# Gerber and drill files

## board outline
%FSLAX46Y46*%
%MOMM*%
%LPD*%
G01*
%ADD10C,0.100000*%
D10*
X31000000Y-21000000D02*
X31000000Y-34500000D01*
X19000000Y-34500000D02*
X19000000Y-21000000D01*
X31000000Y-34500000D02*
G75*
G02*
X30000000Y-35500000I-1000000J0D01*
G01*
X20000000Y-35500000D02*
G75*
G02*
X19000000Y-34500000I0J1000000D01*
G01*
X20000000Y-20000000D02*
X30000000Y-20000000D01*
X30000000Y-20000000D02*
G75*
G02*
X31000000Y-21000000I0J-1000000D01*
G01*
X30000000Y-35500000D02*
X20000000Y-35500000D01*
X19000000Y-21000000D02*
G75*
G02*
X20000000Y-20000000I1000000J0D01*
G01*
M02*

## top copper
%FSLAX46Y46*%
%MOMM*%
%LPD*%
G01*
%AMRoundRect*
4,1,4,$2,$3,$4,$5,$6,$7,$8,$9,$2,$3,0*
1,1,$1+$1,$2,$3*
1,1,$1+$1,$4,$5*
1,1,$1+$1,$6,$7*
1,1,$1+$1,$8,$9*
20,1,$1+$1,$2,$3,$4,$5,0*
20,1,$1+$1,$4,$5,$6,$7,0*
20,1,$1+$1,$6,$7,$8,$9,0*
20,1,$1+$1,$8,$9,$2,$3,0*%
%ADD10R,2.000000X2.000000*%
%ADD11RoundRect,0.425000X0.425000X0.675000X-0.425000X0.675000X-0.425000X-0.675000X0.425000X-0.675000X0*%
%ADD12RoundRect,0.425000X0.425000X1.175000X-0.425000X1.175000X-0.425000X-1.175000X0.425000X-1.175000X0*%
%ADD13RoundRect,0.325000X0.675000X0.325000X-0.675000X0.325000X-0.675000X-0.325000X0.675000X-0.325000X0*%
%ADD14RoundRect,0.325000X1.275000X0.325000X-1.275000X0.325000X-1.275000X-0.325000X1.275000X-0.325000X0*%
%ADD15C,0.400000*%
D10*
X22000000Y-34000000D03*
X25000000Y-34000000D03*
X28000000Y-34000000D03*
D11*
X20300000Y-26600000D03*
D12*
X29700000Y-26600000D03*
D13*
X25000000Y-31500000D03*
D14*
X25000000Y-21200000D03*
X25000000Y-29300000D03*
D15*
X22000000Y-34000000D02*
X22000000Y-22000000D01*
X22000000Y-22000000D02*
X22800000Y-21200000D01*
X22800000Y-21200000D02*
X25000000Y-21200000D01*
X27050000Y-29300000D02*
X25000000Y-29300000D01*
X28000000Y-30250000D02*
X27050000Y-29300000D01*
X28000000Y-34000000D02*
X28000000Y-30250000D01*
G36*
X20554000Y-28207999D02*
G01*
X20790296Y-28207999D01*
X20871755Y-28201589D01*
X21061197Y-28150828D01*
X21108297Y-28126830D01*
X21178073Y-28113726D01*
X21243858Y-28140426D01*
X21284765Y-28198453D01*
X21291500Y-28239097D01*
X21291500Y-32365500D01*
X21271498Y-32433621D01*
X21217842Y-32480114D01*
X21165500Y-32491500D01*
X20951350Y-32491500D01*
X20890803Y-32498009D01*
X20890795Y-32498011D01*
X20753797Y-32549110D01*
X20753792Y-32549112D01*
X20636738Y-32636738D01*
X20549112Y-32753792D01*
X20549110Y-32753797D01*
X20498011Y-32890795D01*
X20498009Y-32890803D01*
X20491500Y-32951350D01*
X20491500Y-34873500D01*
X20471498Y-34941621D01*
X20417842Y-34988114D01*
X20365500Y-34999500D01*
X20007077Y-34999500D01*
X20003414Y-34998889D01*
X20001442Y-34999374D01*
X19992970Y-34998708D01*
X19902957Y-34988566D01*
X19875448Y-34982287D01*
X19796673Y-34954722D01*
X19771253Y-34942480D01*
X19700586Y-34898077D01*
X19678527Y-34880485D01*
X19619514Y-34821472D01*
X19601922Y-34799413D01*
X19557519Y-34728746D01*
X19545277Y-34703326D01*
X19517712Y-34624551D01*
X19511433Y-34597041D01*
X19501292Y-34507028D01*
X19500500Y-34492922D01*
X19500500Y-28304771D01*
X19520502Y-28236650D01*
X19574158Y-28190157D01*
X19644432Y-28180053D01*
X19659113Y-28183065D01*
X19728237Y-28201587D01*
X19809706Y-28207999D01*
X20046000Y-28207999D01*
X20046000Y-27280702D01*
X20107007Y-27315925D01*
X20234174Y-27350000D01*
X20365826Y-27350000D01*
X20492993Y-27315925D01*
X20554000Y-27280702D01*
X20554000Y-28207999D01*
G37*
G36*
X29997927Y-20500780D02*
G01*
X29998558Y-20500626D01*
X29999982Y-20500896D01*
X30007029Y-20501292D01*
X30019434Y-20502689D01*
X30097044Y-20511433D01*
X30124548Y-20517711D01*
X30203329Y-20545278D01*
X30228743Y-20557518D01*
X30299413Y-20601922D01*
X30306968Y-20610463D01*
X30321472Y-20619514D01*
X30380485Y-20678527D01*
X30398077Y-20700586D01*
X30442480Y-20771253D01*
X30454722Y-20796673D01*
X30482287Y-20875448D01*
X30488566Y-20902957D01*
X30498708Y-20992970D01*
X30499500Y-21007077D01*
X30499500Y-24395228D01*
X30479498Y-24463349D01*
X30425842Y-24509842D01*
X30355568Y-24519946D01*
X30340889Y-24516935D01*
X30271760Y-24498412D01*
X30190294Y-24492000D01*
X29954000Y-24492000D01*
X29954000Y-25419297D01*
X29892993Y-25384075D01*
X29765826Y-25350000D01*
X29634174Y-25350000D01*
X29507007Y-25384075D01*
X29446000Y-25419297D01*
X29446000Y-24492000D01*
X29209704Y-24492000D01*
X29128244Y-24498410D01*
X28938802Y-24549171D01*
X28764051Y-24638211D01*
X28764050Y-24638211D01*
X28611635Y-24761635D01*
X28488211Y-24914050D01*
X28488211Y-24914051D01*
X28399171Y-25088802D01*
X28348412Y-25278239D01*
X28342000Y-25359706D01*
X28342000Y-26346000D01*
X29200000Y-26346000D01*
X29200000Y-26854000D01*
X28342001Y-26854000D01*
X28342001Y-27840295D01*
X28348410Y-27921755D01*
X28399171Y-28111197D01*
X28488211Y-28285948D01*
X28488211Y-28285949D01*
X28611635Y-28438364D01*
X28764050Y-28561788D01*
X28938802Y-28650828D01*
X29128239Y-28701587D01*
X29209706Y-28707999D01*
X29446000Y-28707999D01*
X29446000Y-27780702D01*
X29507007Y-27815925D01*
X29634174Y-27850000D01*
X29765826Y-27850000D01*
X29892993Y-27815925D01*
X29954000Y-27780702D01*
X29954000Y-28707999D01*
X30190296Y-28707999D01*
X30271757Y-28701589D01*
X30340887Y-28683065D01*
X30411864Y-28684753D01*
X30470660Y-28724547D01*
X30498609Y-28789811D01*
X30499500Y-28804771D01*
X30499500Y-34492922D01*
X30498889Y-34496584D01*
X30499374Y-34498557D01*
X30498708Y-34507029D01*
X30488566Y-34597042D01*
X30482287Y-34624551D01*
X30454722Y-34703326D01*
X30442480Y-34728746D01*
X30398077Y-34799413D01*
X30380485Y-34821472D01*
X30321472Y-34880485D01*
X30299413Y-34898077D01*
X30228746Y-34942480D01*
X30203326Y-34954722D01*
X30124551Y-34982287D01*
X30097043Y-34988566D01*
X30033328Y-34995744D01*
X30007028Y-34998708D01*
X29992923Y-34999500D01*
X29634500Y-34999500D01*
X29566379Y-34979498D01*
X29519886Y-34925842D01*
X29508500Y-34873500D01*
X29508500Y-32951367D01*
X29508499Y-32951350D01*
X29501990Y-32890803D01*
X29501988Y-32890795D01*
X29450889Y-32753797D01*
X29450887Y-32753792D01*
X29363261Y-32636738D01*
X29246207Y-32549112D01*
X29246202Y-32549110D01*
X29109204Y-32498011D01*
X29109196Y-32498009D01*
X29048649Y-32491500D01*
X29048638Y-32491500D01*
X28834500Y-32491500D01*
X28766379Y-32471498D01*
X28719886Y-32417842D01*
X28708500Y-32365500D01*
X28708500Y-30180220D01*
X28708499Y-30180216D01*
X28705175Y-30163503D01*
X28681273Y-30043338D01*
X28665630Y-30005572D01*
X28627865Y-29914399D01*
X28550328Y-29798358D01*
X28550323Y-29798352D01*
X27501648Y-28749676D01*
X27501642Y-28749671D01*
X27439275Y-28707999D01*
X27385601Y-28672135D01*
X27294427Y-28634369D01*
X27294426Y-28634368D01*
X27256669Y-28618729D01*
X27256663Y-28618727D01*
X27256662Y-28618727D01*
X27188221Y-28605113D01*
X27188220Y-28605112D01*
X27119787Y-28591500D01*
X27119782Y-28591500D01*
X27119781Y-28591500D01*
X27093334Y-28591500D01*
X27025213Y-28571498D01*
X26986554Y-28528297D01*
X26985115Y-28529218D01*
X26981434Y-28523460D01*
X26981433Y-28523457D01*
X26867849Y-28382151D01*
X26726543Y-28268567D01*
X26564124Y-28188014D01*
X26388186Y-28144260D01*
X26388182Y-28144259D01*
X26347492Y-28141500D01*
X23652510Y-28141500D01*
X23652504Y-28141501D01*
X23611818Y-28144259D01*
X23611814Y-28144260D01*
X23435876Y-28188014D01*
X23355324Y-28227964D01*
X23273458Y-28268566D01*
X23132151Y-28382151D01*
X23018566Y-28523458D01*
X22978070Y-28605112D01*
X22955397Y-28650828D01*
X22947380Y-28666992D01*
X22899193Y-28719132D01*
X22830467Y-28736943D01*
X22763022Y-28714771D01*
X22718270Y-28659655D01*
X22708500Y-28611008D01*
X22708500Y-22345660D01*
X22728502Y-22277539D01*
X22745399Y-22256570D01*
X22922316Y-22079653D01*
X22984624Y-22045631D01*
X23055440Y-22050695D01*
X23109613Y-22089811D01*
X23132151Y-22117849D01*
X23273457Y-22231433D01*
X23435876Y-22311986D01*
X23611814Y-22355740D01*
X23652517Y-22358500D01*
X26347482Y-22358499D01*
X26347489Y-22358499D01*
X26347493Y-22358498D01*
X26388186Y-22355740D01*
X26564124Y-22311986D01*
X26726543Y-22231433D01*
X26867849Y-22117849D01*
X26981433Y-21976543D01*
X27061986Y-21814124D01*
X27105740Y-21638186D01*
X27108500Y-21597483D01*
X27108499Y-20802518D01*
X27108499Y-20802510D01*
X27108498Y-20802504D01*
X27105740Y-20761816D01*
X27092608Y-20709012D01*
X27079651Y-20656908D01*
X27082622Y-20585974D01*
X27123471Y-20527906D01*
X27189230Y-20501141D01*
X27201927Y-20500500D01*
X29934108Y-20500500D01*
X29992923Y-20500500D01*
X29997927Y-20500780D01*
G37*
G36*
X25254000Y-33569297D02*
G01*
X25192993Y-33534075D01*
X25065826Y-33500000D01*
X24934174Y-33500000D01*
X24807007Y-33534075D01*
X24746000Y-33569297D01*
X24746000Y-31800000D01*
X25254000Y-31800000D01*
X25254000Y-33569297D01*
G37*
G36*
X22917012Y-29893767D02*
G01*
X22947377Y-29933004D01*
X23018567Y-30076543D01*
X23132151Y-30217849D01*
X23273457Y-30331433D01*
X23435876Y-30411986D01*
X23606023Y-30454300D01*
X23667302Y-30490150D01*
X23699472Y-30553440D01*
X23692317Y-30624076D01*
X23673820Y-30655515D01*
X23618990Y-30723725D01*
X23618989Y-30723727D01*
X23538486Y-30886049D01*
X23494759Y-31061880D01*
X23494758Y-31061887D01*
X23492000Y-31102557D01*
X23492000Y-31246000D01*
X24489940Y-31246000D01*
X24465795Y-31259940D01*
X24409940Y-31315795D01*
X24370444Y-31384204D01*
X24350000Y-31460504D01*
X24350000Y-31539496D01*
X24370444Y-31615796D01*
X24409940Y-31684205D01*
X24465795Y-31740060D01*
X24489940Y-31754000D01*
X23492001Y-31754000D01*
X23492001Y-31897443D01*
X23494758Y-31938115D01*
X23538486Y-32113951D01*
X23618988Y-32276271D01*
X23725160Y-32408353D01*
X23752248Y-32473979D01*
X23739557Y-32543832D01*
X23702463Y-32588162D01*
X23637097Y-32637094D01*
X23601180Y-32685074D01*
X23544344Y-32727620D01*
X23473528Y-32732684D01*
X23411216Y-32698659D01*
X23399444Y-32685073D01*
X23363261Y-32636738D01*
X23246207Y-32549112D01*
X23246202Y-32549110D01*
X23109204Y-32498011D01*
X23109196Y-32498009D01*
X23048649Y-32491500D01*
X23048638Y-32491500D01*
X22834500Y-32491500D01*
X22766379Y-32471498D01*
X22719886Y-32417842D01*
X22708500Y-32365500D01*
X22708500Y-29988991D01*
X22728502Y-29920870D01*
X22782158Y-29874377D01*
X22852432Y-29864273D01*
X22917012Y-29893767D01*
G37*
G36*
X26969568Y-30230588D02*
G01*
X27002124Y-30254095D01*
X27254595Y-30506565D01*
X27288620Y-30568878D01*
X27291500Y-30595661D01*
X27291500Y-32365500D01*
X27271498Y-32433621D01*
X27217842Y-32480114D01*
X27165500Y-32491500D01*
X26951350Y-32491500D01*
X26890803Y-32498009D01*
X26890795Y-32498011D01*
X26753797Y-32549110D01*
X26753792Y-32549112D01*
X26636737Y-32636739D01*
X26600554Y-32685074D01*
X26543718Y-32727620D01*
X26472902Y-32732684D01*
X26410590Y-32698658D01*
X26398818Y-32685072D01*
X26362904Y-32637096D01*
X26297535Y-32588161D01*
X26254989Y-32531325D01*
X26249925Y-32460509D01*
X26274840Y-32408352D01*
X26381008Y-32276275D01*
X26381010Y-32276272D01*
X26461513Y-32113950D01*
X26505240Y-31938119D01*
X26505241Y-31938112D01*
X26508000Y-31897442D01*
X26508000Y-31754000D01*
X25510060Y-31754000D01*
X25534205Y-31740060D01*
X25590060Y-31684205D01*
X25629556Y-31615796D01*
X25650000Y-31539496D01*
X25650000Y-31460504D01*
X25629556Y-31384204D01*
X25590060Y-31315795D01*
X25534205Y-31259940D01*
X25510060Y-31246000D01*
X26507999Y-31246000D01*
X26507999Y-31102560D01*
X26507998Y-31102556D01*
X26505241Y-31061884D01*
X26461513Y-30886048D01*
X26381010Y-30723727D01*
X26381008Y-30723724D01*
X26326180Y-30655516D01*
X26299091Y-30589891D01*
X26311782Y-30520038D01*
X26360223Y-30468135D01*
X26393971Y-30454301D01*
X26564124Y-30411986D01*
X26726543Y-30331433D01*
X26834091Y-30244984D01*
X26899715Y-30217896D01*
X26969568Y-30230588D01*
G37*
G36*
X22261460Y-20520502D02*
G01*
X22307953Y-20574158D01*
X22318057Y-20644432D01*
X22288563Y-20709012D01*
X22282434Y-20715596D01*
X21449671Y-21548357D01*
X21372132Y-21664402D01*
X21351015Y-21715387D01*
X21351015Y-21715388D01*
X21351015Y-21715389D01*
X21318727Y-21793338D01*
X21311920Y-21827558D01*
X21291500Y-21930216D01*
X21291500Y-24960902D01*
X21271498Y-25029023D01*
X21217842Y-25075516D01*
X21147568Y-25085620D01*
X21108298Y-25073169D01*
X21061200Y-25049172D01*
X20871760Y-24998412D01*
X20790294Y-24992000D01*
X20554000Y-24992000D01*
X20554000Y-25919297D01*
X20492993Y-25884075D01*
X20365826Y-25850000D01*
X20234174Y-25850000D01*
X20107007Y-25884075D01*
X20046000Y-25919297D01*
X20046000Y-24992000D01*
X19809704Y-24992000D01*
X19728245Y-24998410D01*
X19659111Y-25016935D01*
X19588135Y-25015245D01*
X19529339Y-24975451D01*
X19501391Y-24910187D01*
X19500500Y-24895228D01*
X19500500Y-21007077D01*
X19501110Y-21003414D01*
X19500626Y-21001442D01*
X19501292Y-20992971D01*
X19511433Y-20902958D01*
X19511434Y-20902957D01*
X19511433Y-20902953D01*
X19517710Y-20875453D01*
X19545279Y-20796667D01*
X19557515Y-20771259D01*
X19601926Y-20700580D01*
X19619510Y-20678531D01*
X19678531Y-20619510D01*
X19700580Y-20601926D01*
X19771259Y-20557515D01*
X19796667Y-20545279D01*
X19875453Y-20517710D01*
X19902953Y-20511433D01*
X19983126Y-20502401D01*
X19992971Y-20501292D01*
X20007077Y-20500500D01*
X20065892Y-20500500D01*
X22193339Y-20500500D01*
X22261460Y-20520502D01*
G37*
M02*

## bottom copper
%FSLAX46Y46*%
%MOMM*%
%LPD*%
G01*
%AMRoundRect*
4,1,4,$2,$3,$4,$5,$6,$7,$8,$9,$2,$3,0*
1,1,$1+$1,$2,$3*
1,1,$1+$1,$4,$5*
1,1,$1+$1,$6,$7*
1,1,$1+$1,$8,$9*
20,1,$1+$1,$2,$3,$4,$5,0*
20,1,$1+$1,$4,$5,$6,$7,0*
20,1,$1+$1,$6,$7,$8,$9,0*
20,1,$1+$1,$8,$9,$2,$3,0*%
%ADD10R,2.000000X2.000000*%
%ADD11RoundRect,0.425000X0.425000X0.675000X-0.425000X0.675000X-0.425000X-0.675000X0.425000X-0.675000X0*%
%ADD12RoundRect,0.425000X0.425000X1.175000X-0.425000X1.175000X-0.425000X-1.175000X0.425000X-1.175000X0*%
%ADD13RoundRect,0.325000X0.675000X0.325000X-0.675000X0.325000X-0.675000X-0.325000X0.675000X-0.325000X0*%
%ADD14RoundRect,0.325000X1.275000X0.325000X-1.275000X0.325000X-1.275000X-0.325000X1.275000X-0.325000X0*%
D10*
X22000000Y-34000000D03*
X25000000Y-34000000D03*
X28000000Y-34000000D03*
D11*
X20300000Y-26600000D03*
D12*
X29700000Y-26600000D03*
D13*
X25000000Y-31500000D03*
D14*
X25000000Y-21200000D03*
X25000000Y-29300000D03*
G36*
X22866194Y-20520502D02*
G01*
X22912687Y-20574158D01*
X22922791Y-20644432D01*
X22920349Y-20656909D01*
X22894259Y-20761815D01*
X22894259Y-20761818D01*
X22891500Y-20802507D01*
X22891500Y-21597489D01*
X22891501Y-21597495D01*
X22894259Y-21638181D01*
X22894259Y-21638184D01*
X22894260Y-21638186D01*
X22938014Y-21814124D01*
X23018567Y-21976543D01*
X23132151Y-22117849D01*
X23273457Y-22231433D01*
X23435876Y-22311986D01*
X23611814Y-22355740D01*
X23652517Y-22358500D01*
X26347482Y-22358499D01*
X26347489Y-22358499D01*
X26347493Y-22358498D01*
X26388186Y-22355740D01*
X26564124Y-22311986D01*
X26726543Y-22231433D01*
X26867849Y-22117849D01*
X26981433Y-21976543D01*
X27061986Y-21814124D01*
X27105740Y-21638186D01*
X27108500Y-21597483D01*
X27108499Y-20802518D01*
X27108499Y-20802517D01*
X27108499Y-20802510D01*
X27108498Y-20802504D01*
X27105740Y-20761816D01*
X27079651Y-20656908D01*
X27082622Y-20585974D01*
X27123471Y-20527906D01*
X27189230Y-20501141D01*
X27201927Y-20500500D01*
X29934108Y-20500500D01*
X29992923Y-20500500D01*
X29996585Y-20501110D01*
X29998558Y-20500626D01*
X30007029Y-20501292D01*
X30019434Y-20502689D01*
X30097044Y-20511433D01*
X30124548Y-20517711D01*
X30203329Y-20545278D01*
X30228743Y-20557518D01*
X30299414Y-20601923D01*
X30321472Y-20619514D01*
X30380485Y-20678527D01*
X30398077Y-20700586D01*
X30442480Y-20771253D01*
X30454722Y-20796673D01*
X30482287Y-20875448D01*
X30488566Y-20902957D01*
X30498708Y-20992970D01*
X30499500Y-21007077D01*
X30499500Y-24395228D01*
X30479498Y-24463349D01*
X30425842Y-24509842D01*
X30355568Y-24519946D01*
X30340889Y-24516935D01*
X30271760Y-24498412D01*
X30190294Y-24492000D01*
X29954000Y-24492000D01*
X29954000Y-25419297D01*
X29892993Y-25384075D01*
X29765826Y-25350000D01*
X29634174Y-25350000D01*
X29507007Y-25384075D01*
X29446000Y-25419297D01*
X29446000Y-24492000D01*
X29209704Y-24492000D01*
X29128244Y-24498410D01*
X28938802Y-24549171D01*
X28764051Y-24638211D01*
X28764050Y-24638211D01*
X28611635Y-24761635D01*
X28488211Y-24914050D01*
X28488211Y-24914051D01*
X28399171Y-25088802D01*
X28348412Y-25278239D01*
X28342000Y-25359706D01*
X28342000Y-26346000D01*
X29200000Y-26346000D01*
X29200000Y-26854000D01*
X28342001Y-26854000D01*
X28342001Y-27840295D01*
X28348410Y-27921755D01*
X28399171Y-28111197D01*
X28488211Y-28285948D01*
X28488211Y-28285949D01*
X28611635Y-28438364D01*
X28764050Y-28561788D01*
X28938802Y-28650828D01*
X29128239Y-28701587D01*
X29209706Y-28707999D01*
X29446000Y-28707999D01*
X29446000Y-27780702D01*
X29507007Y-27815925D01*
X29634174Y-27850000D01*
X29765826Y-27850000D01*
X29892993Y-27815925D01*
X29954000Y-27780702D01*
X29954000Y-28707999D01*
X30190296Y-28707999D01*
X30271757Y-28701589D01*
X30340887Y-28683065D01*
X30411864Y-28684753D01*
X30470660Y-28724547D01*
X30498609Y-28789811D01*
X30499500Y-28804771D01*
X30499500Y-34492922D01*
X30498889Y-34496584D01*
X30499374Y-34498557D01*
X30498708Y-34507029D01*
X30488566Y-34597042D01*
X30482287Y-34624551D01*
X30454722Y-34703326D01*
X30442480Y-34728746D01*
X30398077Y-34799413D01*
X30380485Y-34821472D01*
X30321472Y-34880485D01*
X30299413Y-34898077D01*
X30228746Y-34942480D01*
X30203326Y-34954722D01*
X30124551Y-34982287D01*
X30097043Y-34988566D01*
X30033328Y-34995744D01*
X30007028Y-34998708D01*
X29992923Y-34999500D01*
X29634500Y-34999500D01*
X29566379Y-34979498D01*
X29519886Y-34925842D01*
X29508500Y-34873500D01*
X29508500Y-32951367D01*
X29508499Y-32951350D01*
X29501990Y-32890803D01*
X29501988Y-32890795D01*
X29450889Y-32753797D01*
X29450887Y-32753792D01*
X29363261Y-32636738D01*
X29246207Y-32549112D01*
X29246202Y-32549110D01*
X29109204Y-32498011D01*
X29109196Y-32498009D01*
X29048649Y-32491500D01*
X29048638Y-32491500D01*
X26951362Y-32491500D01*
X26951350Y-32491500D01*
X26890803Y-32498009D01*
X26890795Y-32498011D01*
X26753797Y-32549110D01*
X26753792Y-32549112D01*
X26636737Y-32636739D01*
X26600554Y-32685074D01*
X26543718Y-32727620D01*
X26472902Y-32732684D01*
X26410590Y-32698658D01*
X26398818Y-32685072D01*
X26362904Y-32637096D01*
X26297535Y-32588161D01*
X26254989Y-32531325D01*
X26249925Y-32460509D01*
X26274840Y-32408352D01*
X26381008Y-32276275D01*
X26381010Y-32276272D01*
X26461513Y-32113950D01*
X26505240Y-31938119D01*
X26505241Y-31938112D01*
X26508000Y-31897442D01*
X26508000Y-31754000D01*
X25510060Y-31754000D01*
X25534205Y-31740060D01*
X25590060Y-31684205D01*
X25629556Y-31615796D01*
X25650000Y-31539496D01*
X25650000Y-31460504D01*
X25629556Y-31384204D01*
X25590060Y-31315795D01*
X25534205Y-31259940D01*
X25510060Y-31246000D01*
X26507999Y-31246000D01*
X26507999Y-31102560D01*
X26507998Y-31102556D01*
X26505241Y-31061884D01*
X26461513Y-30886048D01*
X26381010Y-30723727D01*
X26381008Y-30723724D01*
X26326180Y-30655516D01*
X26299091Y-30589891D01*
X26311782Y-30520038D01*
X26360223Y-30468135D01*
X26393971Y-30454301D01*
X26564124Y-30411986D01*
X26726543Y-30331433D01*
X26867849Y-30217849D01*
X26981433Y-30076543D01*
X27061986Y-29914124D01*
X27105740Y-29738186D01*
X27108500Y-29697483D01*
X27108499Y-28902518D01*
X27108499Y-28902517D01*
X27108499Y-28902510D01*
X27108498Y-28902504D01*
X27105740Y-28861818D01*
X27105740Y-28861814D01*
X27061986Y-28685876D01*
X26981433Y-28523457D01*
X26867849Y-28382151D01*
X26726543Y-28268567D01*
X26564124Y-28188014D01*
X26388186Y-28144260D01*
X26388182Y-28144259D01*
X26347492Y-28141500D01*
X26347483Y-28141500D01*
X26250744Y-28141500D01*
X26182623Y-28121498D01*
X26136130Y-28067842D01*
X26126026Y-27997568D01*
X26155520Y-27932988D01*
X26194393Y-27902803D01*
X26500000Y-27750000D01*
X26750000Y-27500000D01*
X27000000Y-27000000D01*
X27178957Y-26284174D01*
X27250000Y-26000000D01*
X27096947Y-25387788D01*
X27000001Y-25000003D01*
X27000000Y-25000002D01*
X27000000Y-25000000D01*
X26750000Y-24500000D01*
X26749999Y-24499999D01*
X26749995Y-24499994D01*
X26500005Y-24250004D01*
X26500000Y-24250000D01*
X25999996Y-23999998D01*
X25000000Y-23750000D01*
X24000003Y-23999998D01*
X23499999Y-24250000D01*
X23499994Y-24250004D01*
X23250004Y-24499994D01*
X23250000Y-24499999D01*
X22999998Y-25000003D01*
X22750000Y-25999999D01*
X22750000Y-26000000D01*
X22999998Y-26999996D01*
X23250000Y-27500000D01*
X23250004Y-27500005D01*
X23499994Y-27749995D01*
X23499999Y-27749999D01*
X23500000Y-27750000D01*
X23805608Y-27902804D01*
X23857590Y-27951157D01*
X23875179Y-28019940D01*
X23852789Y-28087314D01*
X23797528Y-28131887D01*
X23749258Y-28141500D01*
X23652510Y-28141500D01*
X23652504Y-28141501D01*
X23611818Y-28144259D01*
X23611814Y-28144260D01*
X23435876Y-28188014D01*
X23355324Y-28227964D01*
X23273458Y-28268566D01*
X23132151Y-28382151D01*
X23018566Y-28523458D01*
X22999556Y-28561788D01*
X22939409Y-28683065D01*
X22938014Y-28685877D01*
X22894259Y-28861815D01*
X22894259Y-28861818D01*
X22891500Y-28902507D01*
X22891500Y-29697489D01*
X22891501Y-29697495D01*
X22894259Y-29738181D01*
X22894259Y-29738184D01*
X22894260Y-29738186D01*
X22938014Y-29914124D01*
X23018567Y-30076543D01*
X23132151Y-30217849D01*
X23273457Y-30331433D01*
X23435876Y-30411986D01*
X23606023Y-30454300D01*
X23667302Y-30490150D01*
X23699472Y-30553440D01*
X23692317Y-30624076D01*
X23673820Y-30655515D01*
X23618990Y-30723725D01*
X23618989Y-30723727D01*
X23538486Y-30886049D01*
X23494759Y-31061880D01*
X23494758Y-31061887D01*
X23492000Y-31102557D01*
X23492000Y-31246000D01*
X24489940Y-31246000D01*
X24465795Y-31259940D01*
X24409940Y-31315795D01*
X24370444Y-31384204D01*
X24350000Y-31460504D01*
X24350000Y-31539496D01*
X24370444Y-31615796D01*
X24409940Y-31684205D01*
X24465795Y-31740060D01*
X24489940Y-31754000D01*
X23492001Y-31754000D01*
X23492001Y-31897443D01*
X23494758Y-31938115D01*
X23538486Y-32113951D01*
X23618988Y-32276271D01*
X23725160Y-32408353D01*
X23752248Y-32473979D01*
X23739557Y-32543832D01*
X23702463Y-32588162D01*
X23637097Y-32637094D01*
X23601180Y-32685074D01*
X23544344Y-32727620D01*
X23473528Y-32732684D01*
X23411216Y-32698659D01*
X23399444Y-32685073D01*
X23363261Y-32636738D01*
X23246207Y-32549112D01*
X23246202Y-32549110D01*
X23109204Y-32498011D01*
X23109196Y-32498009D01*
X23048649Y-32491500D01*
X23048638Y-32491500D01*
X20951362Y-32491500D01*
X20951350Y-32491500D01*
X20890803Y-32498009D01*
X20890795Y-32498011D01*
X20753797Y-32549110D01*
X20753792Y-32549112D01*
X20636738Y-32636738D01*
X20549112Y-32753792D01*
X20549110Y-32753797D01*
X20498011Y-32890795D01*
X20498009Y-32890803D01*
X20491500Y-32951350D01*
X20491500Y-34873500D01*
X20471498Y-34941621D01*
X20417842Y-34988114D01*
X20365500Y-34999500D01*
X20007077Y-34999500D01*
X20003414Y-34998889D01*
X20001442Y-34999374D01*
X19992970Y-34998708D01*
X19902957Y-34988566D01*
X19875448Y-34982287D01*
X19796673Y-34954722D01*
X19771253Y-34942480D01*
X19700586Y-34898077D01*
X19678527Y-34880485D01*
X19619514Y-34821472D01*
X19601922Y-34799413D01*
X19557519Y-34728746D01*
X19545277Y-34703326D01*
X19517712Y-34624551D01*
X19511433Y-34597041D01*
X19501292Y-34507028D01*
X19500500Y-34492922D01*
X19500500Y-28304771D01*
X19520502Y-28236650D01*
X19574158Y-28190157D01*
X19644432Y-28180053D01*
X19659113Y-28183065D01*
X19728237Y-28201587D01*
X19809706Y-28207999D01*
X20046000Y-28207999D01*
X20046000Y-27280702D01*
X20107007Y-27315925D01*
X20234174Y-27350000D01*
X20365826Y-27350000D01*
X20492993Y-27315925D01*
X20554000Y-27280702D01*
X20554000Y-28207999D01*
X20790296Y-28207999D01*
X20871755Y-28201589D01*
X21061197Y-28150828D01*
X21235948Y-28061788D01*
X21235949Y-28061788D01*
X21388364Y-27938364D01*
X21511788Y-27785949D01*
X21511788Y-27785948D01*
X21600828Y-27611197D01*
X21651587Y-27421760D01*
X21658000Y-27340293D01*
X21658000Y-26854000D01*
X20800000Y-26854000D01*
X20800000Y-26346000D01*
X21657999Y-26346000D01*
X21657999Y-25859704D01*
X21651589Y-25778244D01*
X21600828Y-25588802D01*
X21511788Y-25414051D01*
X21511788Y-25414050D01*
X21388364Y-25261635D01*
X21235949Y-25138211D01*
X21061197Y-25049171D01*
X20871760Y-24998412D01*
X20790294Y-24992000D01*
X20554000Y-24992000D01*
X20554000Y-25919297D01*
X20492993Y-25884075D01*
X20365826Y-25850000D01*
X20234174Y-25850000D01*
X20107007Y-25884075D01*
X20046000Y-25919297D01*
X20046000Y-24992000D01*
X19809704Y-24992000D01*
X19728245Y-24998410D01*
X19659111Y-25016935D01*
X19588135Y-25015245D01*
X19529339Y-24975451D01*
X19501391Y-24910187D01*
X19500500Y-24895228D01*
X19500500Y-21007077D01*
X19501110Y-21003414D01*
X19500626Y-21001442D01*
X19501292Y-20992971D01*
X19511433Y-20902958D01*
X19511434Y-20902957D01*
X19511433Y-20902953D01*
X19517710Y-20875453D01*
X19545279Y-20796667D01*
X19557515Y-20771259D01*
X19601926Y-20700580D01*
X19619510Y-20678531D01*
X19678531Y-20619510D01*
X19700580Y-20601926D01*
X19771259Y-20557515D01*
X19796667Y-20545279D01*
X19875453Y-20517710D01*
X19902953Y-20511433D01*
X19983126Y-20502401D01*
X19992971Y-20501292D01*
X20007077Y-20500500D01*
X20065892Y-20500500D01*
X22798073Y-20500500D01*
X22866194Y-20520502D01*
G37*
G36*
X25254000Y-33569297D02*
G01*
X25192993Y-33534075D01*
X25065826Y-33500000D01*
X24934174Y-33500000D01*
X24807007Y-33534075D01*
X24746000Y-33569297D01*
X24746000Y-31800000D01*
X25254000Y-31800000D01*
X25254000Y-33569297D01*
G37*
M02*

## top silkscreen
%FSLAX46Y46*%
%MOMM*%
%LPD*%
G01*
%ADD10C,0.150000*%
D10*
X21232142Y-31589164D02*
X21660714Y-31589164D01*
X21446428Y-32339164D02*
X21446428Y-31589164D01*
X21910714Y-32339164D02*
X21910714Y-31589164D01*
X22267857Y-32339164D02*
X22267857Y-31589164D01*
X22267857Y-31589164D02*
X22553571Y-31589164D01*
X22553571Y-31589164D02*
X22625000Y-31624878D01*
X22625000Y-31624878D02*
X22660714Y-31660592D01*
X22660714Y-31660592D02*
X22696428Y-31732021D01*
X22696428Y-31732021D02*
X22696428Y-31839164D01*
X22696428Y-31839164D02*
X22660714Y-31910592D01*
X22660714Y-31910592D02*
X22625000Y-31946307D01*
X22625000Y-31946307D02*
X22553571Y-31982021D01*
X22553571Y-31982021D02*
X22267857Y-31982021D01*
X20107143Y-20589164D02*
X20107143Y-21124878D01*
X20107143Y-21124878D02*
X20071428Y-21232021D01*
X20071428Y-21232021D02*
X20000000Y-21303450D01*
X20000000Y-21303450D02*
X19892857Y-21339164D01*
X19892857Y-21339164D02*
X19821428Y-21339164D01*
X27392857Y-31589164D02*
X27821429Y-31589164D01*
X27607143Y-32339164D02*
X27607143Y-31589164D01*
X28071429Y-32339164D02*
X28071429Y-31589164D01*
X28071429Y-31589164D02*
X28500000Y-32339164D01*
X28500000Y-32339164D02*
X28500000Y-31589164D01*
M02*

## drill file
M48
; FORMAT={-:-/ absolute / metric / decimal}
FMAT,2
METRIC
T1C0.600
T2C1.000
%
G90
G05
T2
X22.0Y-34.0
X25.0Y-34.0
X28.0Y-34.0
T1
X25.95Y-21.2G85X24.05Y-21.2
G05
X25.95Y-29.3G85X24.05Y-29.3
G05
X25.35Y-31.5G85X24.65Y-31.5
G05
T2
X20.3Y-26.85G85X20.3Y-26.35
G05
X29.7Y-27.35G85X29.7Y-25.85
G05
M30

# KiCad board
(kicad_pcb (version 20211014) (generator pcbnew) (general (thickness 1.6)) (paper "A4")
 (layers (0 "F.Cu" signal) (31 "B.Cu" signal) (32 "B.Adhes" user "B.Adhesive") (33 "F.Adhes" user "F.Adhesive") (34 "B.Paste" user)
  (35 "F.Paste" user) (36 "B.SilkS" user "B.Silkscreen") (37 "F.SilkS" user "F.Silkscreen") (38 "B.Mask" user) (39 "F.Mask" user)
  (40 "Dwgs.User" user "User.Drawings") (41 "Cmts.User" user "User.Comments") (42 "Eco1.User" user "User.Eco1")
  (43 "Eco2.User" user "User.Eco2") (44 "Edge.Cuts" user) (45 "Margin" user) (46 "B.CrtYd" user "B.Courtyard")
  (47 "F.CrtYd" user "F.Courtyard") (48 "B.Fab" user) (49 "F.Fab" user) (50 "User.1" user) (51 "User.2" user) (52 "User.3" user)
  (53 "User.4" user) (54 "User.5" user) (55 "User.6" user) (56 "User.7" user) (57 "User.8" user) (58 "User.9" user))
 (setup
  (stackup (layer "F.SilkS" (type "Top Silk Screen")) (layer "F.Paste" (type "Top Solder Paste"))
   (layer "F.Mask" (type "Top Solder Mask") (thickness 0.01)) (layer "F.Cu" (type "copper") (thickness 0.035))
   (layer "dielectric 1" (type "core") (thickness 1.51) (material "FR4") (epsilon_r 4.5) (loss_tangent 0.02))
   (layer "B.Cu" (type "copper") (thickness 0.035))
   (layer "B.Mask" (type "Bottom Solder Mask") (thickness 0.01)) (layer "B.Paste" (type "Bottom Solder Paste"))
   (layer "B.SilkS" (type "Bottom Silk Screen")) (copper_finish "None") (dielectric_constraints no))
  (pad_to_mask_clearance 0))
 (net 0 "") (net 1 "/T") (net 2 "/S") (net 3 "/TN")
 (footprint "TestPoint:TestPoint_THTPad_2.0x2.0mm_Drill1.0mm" (layer "B.Cu") (at 22 34 180)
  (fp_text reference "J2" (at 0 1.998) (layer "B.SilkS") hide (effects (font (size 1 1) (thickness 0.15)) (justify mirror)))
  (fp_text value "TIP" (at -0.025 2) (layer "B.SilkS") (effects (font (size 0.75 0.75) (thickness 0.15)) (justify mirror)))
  (pad "1" thru_hole rect locked (at 0 0 180) (size 2 2) (drill 1) (layers *.Cu *.Mask) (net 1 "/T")))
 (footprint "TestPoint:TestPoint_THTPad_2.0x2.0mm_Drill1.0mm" (layer "B.Cu") (at 25 34 180)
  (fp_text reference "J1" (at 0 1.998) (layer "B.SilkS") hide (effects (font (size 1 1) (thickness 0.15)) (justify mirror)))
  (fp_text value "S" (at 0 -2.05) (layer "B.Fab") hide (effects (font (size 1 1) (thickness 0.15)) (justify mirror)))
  (pad "1" thru_hole rect locked (at 0 0 180) (size 2 2) (drill 1) (layers *.Cu *.Mask) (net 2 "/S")))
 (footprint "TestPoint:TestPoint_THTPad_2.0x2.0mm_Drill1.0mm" (layer "B.Cu") (at 28 34 180)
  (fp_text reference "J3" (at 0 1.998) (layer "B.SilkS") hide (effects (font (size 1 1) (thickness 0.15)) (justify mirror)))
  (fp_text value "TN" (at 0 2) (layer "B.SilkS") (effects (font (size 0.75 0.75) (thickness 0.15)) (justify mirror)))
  (pad "1" thru_hole rect locked (at 0 0 180) (size 2 2) (drill 1) (layers *.Cu *.Mask) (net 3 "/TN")))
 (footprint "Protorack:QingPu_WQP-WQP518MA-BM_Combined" (layer "B.Cu") (at 25 26 180)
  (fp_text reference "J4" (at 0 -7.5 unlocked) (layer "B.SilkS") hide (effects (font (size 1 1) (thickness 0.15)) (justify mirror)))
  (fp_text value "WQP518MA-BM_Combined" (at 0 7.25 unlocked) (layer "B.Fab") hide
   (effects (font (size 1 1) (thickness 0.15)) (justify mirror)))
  (pad "S" thru_hole roundrect (at 4.7 -0.6 180) (size 1.7 2.2) (drill oval 1 1.5) (layers *.Cu *.Mask) (roundrect_rratio 0.25) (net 2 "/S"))
  (pad "S" thru_hole roundrect (at -4.7 -0.6 180) (size 1.7 3.2) (drill oval 1 2.5) (layers *.Cu *.Mask) (roundrect_rratio 0.25)
   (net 2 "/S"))
  (pad "S" thru_hole roundrect (at 0 -5.5 180) (size 2 1.3) (drill oval 1.3 0.6) (layers *.Cu *.Mask) (roundrect_rratio 0.25) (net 2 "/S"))
  (pad "T" thru_hole roundrect (at 0 4.8 180) (size 3.2 1.3) (drill oval 2.5 0.6) (layers *.Cu *.Mask) (roundrect_rratio 0.25) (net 1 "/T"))
  (pad "TN" thru_hole roundrect (at 0 -3.3 180) (size 3.2 1.3) (drill oval 2.5 0.6) (layers *.Cu *.Mask) (roundrect_rratio 0.25)
   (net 3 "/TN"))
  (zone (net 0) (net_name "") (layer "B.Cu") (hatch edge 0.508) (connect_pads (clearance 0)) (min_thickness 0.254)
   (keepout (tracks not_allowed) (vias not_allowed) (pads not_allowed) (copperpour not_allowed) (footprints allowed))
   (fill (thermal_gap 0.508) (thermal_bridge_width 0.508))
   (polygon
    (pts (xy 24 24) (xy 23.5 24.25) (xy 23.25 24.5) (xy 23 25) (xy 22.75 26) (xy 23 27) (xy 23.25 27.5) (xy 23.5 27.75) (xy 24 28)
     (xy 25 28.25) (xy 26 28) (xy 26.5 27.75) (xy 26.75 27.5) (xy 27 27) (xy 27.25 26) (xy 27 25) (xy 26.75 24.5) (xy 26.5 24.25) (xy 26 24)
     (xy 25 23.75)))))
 (gr_line (start 31 21) (end 31 34.5) (layer "Edge.Cuts") (width 0.1))
 (gr_line (start 19 34.5) (end 19 21) (layer "Edge.Cuts") (width 0.1))
 (gr_arc (start 31 34.5) (mid 30.707107 35.207107) (end 30 35.5) (layer "Edge.Cuts") (width 0.1))
 (gr_arc (start 20 35.5) (mid 19.292893 35.207107) (end 19 34.5) (layer "Edge.Cuts") (width 0.1))
 (gr_line (start 20 20) (end 30 20) (layer "Edge.Cuts") (width 0.1))
 (gr_arc (start 30 20) (mid 30.707107 20.292893) (end 31 21) (layer "Edge.Cuts") (width 0.1))
 (gr_line (start 30 35.5) (end 20 35.5) (layer "Edge.Cuts") (width 0.1))
 (gr_arc (start 19 21) (mid 19.292893 20.292893) (end 20 20) (layer "Edge.Cuts") (width 0.1))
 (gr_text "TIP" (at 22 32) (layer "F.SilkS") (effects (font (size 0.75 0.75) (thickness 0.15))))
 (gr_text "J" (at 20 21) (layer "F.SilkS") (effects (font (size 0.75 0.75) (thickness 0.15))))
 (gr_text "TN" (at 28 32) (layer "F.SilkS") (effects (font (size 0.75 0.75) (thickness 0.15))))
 (segment (start 22 34) (end 22 22) (width 0.4) (layer "F.Cu") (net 1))
 (segment (start 22 22) (end 22.8 21.2) (width 0.4) (layer "F.Cu") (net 1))
 (segment (start 22.8 21.2) (end 25 21.2) (width 0.4) (layer "F.Cu") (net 1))
 (segment (start 27.05 29.3) (end 25 29.3) (width 0.4) (layer "F.Cu") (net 3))
 (segment (start 28 30.25) (end 27.05 29.3) (width 0.4) (layer "F.Cu") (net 3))
 (segment (start 28 34) (end 28 30.25) (width 0.4) (layer "F.Cu") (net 3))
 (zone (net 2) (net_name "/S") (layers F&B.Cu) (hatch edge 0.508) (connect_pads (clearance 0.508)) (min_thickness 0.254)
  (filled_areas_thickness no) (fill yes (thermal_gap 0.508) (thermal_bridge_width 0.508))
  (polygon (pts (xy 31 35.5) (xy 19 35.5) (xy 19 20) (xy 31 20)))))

